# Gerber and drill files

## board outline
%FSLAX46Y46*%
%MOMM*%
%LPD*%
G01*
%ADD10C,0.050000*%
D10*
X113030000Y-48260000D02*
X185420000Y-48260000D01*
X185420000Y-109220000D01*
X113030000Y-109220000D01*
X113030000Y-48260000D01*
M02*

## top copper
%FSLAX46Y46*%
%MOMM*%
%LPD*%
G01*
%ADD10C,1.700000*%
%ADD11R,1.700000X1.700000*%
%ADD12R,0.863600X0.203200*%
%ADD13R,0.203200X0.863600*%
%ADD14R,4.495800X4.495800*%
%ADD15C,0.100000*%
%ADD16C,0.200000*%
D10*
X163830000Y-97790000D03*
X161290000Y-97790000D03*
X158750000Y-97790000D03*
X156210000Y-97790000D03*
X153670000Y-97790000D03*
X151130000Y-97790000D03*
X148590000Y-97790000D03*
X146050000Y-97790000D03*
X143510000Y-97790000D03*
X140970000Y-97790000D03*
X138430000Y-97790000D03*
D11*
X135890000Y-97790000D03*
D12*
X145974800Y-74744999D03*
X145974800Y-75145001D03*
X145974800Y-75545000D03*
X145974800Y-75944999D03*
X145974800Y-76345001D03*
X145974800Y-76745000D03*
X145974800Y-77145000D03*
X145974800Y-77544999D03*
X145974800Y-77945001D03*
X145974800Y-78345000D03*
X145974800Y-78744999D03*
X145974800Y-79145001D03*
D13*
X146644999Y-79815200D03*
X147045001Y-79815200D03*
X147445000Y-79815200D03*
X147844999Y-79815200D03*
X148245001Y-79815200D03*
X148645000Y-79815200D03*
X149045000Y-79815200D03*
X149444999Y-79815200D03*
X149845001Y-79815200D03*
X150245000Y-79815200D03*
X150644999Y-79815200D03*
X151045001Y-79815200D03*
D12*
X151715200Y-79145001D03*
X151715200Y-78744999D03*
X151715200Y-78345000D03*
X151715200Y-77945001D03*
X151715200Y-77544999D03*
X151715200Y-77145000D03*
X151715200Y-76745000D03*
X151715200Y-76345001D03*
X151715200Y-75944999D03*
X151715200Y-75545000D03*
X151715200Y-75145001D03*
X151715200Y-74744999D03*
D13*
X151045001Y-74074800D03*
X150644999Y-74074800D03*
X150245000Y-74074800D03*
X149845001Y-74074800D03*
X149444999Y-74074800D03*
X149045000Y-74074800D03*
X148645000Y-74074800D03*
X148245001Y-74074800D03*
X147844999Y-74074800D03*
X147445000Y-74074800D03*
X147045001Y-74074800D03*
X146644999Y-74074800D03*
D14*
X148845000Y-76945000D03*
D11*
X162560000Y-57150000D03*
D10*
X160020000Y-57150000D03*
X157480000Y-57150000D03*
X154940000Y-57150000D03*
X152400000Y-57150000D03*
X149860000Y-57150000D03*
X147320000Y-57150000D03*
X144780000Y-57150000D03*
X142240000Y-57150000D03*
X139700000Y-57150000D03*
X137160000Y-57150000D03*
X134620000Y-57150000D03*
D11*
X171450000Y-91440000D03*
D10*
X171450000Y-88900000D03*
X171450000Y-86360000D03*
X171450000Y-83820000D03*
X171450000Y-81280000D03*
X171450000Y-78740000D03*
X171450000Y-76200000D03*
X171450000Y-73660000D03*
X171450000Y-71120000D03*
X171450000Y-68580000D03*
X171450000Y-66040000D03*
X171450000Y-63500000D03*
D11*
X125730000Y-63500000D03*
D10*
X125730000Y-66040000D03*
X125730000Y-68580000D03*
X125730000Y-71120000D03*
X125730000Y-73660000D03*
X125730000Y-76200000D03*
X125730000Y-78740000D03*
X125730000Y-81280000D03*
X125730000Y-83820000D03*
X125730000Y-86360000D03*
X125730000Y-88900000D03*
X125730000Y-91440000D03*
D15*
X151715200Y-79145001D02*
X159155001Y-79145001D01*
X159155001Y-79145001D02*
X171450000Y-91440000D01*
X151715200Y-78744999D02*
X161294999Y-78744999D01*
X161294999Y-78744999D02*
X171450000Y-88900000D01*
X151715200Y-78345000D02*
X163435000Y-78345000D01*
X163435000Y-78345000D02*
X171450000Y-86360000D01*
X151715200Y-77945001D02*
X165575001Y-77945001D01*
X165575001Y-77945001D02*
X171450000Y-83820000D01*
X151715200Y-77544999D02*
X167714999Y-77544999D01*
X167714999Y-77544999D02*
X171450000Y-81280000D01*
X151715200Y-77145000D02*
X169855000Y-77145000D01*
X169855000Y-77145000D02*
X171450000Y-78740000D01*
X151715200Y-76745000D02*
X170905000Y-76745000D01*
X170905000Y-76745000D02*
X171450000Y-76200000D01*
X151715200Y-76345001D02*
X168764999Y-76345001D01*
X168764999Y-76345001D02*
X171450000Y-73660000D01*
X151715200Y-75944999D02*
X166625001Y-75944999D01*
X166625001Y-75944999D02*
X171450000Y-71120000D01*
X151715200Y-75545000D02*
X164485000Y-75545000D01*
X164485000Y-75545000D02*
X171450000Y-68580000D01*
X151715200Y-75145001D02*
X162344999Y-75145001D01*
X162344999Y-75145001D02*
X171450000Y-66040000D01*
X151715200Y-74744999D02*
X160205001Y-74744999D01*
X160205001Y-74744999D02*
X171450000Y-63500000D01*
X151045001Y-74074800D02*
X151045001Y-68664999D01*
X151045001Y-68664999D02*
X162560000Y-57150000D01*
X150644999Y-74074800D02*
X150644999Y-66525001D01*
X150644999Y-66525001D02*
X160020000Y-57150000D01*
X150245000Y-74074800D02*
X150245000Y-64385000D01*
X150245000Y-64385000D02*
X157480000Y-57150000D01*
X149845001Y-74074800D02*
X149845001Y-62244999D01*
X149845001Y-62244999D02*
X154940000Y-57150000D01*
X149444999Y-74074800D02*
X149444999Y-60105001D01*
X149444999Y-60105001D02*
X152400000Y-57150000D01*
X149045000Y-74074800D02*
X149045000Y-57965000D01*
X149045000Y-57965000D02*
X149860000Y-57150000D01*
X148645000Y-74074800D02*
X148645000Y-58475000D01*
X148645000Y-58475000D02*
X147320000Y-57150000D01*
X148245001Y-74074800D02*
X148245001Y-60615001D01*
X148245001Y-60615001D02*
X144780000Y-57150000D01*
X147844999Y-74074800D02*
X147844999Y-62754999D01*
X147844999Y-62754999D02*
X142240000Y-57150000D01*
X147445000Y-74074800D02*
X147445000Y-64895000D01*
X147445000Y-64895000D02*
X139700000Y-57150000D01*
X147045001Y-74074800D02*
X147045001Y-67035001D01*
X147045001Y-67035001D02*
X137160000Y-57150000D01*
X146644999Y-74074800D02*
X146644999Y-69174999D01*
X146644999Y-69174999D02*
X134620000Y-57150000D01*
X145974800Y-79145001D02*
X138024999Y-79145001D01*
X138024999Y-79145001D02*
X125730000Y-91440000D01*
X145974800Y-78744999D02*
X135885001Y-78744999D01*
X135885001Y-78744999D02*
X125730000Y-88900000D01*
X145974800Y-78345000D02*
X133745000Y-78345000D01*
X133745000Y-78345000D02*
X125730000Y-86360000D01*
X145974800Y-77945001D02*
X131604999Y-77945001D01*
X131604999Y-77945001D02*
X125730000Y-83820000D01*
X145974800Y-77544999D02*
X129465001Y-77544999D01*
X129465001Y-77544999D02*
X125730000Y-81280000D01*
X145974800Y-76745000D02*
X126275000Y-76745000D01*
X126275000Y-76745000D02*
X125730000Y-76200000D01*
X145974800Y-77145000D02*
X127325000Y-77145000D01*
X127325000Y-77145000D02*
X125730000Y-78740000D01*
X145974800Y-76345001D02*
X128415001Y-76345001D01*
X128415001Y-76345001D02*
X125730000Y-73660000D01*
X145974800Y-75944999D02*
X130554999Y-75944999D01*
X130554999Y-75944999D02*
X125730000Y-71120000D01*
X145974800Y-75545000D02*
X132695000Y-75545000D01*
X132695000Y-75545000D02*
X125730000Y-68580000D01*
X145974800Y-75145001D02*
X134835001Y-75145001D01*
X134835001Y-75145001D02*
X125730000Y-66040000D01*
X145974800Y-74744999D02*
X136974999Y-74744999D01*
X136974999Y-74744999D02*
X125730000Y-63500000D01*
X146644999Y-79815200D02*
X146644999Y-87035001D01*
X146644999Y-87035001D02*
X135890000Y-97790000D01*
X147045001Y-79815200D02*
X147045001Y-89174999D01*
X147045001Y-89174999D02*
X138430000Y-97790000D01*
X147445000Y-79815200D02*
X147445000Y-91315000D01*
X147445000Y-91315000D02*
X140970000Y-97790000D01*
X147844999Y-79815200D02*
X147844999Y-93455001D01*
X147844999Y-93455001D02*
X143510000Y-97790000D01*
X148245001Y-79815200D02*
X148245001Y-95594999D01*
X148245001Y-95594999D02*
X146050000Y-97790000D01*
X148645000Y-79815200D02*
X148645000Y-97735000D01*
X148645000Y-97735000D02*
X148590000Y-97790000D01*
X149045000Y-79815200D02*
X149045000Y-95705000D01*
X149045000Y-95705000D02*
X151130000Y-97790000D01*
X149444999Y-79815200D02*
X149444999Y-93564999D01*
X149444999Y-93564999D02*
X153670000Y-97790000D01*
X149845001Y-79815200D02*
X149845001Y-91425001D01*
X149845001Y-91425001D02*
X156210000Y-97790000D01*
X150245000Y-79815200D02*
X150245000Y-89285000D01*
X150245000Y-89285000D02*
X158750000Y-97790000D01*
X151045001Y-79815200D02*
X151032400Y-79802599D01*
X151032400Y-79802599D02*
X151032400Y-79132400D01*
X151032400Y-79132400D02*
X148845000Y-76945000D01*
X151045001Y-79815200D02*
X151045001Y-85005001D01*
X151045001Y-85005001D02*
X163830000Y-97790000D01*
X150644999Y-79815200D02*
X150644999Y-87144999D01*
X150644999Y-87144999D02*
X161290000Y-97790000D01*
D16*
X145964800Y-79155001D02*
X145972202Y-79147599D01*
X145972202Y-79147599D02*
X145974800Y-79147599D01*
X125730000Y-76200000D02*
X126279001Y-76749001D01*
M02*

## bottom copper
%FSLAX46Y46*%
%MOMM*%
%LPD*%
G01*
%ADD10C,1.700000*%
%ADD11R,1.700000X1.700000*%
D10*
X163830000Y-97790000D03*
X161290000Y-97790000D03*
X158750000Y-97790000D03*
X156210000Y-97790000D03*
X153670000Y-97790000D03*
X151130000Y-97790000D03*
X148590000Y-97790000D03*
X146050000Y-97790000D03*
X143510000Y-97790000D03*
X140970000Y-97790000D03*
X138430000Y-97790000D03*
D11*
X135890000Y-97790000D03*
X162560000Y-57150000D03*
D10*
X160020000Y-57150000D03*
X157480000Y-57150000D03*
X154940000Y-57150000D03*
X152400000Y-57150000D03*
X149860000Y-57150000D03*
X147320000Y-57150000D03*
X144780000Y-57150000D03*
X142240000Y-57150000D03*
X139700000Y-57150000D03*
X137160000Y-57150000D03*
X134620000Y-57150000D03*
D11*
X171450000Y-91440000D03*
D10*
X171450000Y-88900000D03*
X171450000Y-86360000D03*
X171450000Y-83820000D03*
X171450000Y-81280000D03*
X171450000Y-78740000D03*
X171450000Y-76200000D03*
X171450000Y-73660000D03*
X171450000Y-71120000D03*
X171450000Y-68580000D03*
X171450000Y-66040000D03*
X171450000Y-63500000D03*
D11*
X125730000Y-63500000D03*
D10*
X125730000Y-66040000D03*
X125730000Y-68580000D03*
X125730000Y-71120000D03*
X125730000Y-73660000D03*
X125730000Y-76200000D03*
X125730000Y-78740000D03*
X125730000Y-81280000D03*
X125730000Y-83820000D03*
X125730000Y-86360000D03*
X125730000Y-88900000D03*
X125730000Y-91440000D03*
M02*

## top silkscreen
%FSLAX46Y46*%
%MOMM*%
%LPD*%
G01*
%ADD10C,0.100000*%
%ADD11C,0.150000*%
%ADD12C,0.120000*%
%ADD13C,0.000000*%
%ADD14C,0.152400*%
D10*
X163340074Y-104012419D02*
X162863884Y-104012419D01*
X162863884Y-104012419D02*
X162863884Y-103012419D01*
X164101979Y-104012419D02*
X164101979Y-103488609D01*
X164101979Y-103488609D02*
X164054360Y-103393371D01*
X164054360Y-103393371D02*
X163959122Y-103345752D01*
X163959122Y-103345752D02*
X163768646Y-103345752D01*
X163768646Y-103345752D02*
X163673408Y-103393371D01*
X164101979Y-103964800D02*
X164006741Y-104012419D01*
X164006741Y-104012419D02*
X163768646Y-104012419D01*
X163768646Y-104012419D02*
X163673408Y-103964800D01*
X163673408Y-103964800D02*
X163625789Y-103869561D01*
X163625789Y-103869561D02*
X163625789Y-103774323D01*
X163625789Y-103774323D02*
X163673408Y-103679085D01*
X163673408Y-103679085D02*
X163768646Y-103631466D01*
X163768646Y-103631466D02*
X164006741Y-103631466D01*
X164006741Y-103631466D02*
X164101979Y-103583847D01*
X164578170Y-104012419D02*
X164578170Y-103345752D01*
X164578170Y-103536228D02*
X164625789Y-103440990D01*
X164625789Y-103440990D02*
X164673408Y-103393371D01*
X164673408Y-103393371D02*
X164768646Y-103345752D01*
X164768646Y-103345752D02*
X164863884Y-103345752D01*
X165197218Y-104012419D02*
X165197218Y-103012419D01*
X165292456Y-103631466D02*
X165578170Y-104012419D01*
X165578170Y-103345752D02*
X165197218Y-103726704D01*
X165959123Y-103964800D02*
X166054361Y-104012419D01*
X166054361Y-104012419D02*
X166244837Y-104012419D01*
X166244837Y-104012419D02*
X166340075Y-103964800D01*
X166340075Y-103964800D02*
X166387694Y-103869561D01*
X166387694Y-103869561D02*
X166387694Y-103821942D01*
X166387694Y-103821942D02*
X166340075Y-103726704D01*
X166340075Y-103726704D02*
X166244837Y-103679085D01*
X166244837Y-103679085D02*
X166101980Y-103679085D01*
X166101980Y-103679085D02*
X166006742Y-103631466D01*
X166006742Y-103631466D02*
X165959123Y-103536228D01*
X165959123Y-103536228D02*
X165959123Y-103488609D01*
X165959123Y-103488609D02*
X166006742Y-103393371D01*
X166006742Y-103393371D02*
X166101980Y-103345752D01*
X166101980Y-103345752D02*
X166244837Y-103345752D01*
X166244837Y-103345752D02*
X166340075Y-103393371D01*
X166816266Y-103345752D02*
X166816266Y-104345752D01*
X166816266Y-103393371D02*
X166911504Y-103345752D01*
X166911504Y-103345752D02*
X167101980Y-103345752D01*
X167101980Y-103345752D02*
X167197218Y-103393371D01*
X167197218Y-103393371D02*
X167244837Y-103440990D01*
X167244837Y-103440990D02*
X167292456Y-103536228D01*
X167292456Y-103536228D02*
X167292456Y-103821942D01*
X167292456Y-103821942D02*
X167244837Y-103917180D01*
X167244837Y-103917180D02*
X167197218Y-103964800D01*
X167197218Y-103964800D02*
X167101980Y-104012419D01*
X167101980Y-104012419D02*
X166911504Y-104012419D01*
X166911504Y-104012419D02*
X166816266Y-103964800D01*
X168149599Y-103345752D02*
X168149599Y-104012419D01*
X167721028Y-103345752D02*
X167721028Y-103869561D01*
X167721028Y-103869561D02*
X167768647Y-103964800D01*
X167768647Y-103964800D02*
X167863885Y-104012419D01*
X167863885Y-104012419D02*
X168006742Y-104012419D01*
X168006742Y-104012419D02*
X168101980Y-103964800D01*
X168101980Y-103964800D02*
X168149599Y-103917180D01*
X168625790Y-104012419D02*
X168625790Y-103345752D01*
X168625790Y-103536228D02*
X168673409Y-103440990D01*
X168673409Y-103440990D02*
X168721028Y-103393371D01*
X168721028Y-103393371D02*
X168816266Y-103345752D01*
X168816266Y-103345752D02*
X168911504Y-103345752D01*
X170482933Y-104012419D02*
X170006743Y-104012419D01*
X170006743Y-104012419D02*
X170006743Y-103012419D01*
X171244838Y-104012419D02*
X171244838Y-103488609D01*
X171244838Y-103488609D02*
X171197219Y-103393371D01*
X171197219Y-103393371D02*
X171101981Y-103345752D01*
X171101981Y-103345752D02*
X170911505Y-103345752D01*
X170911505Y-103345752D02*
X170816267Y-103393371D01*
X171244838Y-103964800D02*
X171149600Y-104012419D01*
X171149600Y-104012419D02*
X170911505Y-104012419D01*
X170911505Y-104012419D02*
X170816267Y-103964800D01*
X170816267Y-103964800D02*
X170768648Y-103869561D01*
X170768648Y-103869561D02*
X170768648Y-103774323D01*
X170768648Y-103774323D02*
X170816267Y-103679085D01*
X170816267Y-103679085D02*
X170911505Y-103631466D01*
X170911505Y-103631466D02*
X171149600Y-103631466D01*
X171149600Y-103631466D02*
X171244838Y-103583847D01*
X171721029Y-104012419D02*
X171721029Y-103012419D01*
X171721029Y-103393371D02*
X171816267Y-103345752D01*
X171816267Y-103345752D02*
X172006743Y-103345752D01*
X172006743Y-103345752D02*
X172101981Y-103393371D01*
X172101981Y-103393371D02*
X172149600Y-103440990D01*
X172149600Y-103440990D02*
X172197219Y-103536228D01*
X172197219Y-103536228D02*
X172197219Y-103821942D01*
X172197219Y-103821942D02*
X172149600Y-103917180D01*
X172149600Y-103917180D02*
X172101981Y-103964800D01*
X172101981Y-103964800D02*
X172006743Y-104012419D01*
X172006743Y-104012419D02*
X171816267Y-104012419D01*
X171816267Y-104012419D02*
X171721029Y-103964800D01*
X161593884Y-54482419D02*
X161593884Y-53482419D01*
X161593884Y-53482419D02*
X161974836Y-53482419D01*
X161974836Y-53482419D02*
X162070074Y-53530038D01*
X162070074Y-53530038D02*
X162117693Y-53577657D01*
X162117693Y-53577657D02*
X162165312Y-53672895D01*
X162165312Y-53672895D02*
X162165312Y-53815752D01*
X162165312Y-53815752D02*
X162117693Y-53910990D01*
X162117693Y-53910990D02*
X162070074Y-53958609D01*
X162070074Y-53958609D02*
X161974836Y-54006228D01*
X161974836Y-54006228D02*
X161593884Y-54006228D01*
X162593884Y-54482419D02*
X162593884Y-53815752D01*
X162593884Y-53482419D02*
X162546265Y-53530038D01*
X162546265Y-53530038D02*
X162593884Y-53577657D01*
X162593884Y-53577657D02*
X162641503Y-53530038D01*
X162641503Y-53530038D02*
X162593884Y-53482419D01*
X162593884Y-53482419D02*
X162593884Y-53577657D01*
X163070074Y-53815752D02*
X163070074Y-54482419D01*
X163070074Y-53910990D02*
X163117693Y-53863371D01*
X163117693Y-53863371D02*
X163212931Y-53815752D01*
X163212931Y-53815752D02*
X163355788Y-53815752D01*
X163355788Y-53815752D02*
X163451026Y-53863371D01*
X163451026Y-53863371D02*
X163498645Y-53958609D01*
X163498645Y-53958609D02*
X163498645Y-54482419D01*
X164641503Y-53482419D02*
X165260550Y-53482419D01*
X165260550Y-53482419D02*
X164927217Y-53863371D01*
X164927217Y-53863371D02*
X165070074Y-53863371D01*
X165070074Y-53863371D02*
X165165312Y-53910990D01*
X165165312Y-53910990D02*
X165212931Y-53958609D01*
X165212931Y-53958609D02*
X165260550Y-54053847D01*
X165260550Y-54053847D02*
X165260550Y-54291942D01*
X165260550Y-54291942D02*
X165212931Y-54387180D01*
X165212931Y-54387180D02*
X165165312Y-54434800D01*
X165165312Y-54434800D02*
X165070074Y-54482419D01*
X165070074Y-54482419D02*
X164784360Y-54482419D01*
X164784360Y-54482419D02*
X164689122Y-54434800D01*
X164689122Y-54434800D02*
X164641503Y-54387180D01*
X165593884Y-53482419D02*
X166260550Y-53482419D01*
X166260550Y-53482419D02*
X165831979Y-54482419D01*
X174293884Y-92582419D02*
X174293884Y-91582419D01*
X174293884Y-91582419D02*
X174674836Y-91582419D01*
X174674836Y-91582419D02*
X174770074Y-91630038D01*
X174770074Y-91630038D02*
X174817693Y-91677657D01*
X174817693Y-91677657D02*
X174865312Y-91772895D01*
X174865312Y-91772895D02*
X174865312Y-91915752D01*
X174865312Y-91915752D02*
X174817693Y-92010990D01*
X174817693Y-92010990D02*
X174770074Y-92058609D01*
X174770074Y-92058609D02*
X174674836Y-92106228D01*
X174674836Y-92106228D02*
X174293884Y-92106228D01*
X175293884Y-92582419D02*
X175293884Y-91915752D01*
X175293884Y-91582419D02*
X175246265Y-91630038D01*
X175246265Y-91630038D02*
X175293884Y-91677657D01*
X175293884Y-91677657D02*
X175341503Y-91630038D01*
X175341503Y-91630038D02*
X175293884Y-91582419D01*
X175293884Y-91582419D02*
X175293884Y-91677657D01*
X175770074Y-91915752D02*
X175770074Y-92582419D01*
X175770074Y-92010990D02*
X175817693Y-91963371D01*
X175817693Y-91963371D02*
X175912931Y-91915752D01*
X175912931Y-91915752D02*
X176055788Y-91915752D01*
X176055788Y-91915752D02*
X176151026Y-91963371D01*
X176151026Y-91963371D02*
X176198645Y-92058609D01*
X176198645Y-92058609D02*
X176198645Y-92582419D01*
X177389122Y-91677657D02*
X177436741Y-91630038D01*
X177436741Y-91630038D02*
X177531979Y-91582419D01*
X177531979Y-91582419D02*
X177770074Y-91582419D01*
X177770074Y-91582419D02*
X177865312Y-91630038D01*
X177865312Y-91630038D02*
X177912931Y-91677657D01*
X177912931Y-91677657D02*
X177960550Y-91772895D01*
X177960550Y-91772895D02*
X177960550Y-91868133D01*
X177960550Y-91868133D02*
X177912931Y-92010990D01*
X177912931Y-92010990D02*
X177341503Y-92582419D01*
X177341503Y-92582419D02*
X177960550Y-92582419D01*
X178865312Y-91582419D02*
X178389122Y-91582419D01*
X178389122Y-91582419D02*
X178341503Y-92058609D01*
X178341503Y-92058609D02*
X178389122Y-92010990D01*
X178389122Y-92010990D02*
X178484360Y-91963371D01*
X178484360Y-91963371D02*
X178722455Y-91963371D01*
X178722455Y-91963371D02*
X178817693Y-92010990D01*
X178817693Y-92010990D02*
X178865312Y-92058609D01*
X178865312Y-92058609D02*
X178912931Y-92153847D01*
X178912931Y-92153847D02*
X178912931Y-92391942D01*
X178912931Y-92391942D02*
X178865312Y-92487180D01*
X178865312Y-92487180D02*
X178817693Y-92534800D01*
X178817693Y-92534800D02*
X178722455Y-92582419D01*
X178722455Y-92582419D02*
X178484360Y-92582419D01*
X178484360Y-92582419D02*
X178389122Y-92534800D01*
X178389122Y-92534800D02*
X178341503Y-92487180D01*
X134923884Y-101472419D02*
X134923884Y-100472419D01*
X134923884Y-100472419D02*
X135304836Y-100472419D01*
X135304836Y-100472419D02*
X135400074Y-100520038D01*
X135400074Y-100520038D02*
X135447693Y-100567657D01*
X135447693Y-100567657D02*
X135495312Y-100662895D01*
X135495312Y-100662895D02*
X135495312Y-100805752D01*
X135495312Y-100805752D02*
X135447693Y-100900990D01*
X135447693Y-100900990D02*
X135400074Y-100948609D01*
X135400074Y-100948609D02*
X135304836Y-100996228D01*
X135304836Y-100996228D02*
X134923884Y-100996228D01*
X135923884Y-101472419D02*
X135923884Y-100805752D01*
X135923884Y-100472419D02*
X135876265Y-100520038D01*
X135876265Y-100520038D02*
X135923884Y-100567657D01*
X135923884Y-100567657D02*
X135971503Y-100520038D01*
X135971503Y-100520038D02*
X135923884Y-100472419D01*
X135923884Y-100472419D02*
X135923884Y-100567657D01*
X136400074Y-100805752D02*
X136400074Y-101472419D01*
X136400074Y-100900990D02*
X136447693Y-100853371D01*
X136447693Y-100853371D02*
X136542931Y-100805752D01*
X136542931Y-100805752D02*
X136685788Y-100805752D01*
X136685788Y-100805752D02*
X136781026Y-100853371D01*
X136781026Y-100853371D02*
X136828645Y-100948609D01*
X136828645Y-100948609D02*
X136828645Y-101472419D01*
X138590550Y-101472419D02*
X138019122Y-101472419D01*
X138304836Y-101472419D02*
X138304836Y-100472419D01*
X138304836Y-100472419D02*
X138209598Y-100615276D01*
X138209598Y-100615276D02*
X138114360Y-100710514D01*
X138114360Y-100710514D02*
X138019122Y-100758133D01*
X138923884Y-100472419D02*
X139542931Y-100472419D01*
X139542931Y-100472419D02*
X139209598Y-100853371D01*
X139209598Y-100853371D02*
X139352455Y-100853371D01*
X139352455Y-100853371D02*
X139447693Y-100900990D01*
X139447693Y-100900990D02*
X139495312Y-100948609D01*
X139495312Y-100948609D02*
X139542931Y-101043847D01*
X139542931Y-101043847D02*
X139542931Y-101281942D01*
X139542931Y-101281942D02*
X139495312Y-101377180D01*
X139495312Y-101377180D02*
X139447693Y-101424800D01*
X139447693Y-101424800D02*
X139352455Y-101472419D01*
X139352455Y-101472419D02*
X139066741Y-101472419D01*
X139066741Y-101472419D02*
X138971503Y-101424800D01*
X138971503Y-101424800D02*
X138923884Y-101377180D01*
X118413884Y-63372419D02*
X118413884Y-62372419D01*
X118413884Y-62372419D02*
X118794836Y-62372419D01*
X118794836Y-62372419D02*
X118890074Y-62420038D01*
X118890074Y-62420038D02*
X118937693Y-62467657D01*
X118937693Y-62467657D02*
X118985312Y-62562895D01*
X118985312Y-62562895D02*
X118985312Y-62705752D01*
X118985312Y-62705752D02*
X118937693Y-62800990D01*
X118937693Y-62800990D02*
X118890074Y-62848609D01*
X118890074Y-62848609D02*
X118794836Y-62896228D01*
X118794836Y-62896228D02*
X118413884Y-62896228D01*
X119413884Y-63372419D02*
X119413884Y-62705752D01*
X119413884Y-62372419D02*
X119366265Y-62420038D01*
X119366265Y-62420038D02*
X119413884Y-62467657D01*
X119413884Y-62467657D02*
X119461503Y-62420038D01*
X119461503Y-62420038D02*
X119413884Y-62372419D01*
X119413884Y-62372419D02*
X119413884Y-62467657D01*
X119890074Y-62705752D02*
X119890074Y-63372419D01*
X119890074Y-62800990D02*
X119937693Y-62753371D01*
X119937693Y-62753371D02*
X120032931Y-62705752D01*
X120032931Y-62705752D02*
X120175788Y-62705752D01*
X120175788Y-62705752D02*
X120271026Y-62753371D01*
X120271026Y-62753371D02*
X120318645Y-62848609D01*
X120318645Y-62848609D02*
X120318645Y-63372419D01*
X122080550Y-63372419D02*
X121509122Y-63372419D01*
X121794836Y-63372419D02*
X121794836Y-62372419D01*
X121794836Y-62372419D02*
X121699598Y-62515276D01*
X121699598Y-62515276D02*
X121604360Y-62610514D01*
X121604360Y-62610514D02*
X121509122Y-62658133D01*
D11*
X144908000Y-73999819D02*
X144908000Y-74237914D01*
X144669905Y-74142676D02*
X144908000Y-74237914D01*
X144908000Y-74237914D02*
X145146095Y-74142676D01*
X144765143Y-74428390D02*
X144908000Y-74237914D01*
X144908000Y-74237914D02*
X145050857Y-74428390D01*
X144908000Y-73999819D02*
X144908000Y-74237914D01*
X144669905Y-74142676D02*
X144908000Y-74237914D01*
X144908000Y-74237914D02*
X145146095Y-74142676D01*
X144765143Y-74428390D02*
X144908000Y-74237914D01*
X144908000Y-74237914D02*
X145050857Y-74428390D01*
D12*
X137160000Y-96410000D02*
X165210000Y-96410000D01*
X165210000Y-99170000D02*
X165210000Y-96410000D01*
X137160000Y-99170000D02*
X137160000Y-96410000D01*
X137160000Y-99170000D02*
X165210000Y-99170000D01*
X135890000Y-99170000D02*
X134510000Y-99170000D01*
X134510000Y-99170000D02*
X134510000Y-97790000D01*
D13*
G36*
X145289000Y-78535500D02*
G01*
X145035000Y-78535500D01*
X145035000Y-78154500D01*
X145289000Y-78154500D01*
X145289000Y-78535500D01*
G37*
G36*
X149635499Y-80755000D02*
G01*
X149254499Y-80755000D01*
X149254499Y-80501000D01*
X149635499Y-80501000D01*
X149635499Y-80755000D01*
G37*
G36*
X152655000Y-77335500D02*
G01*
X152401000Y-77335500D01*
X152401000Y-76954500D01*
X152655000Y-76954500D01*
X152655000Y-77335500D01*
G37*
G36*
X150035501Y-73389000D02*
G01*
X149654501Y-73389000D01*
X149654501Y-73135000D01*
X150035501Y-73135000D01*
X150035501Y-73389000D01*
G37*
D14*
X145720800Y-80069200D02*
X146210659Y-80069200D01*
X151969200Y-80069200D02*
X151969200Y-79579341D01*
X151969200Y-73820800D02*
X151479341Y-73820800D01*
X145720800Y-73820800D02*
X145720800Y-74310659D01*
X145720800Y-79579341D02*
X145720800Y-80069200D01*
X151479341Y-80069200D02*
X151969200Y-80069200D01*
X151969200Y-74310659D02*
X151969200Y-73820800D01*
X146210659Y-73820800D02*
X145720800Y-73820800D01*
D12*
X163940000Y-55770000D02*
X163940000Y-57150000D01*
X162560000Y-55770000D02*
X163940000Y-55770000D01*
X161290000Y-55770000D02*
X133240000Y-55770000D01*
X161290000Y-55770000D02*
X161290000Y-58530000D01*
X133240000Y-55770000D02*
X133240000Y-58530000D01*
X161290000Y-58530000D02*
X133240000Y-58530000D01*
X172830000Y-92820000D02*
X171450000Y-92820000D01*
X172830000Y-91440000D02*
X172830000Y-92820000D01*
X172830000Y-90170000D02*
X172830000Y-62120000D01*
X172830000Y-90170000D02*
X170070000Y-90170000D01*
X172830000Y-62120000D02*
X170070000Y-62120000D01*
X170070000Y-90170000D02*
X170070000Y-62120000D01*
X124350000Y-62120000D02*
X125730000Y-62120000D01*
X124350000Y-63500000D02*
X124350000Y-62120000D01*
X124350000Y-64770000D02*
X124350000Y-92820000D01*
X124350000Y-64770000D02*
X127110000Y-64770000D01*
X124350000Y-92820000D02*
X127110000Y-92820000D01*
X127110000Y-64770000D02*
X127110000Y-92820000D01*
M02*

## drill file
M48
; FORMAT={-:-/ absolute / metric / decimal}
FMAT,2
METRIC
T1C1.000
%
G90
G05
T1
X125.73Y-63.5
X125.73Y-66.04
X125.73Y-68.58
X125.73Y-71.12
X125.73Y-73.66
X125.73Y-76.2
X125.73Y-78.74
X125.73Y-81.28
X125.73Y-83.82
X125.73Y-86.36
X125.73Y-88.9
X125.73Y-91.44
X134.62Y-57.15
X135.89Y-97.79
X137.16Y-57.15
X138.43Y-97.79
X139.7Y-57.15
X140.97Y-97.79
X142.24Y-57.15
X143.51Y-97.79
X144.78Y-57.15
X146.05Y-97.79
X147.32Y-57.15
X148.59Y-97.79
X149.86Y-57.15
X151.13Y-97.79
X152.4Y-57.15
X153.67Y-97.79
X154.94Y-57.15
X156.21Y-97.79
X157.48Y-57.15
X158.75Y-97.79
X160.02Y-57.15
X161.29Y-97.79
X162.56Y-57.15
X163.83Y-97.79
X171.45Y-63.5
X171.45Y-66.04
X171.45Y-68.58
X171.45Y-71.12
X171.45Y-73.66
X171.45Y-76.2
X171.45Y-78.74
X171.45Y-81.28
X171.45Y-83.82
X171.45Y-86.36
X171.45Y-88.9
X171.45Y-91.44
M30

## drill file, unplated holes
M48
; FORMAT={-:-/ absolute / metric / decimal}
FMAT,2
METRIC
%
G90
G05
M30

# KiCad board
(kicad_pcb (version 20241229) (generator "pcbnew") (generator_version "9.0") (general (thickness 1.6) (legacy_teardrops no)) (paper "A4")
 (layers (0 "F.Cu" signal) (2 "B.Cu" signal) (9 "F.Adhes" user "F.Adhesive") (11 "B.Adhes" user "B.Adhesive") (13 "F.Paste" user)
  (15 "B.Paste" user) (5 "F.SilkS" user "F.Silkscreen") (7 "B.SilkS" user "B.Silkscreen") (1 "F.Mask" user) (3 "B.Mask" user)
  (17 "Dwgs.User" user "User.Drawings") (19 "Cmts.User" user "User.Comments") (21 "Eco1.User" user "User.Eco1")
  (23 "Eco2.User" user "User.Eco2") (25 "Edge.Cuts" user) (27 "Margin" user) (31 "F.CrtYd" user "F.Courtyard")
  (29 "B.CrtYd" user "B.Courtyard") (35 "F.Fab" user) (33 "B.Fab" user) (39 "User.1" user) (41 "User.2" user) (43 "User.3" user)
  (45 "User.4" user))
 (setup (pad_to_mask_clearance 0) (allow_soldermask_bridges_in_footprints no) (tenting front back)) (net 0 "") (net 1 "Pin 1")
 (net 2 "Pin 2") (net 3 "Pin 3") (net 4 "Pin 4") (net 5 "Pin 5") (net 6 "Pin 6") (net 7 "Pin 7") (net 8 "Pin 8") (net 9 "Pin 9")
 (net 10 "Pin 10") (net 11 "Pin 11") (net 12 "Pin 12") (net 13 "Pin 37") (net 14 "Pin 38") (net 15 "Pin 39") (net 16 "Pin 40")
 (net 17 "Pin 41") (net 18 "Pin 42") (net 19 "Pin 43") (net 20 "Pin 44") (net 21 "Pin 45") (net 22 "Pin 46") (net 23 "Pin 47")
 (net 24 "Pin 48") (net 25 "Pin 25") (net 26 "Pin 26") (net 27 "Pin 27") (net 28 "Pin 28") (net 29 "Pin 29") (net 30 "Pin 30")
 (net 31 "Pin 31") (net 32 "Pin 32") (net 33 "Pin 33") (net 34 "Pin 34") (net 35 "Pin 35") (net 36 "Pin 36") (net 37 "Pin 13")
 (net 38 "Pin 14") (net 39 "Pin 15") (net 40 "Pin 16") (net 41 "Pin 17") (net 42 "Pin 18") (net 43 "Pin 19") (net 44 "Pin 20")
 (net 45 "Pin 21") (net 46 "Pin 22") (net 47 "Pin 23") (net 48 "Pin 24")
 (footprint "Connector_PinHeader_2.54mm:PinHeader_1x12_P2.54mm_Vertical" (layer "F.Cu") (at 125.73 63.5)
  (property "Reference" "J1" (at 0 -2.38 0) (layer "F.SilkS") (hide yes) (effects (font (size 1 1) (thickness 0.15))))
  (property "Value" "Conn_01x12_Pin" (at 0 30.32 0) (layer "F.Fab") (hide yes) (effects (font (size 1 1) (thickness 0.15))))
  (fp_line (start -1.38 -1.38) (end 0 -1.38) (stroke (width 0.12) (type solid)) (layer "F.SilkS"))
  (fp_line (start -1.38 0) (end -1.38 -1.38) (stroke (width 0.12) (type solid)) (layer "F.SilkS"))
  (fp_line (start -1.38 1.27) (end -1.38 29.32) (stroke (width 0.12) (type solid)) (layer "F.SilkS"))
  (fp_line (start -1.38 1.27) (end 1.38 1.27) (stroke (width 0.12) (type solid)) (layer "F.SilkS"))
  (fp_line (start -1.38 29.32) (end 1.38 29.32) (stroke (width 0.12) (type solid)) (layer "F.SilkS"))
  (fp_line (start 1.38 1.27) (end 1.38 29.32) (stroke (width 0.12) (type solid)) (layer "F.SilkS"))
  (pad "1" thru_hole rect (at 0 0) (size 1.7 1.7) (drill 1) (layers "*.Cu" "*.Mask") (remove_unused_layers no) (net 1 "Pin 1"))
  (pad "2" thru_hole circle (at 0 2.54) (size 1.7 1.7) (drill 1) (layers "*.Cu" "*.Mask") (remove_unused_layers no) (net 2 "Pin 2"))
  (pad "3" thru_hole circle (at 0 5.08) (size 1.7 1.7) (drill 1) (layers "*.Cu" "*.Mask") (remove_unused_layers no) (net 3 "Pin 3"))
  (pad "4" thru_hole circle (at 0 7.62) (size 1.7 1.7) (drill 1) (layers "*.Cu" "*.Mask") (remove_unused_layers no) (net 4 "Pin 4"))
  (pad "5" thru_hole circle (at 0 10.16) (size 1.7 1.7) (drill 1) (layers "*.Cu" "*.Mask") (remove_unused_layers no) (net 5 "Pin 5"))
  (pad "6" thru_hole circle (at 0 12.7) (size 1.7 1.7) (drill 1) (layers "*.Cu" "*.Mask") (remove_unused_layers no) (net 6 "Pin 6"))
  (pad "7" thru_hole circle (at 0 15.24) (size 1.7 1.7) (drill 1) (layers "*.Cu" "*.Mask") (remove_unused_layers no) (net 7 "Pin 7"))
  (pad "8" thru_hole circle (at 0 17.78) (size 1.7 1.7) (drill 1) (layers "*.Cu" "*.Mask") (remove_unused_layers no) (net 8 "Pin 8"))
  (pad "9" thru_hole circle (at 0 20.32) (size 1.7 1.7) (drill 1) (layers "*.Cu" "*.Mask") (remove_unused_layers no) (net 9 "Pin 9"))
  (pad "10" thru_hole circle (at 0 22.86) (size 1.7 1.7) (drill 1) (layers "*.Cu" "*.Mask") (remove_unused_layers no) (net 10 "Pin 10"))
  (pad "11" thru_hole circle (at 0 25.4) (size 1.7 1.7) (drill 1) (layers "*.Cu" "*.Mask") (remove_unused_layers no) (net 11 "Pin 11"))
  (pad "12" thru_hole circle (at 0 27.94) (size 1.7 1.7) (drill 1) (layers "*.Cu" "*.Mask") (remove_unused_layers no) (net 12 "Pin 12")))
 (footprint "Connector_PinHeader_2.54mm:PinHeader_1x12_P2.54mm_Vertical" (layer "F.Cu") (at 162.56 57.15 -90)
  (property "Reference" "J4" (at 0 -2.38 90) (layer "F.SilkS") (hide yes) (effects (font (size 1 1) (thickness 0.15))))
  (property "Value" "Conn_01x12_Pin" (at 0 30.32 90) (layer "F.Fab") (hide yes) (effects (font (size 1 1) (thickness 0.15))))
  (fp_line (start -1.38 29.32) (end 1.38 29.32) (stroke (width 0.12) (type solid)) (layer "F.SilkS"))
  (fp_line (start -1.38 1.27) (end -1.38 29.32) (stroke (width 0.12) (type solid)) (layer "F.SilkS"))
  (fp_line (start -1.38 1.27) (end 1.38 1.27) (stroke (width 0.12) (type solid)) (layer "F.SilkS"))
  (fp_line (start 1.38 1.27) (end 1.38 29.32) (stroke (width 0.12) (type solid)) (layer "F.SilkS"))
  (fp_line (start -1.38 0) (end -1.38 -1.38) (stroke (width 0.12) (type solid)) (layer "F.SilkS"))
  (fp_line (start -1.38 -1.38) (end 0 -1.38) (stroke (width 0.12) (type solid)) (layer "F.SilkS"))
  (pad "1" thru_hole rect (at 0 0 270) (size 1.7 1.7) (drill 1) (layers "*.Cu" "*.Mask") (remove_unused_layers no) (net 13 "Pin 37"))
  (pad "2" thru_hole circle (at 0 2.54 270) (size 1.7 1.7) (drill 1) (layers "*.Cu" "*.Mask") (remove_unused_layers no) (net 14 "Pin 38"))
  (pad "3" thru_hole circle (at 0 5.08 270) (size 1.7 1.7) (drill 1) (layers "*.Cu" "*.Mask") (remove_unused_layers no) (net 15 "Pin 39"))
  (pad "4" thru_hole circle (at 0 7.62 270) (size 1.7 1.7) (drill 1) (layers "*.Cu" "*.Mask") (remove_unused_layers no) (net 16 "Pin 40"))
  (pad "5" thru_hole circle (at 0 10.16 270) (size 1.7 1.7) (drill 1) (layers "*.Cu" "*.Mask") (remove_unused_layers no) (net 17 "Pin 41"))
  (pad "6" thru_hole circle (at 0 12.7 270) (size 1.7 1.7) (drill 1) (layers "*.Cu" "*.Mask") (remove_unused_layers no) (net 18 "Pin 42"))
  (pad "7" thru_hole circle (at 0 15.24 270) (size 1.7 1.7) (drill 1) (layers "*.Cu" "*.Mask") (remove_unused_layers no) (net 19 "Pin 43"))
  (pad "8" thru_hole circle (at 0 17.78 270) (size 1.7 1.7) (drill 1) (layers "*.Cu" "*.Mask") (remove_unused_layers no) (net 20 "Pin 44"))
  (pad "9" thru_hole circle (at 0 20.32 270) (size 1.7 1.7) (drill 1) (layers "*.Cu" "*.Mask") (remove_unused_layers no) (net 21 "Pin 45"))
  (pad "10" thru_hole circle (at 0 22.86 270) (size 1.7 1.7) (drill 1) (layers "*.Cu" "*.Mask") (remove_unused_layers no) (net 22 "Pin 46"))
  (pad "11" thru_hole circle (at 0 25.4 270) (size 1.7 1.7) (drill 1) (layers "*.Cu" "*.Mask") (remove_unused_layers no) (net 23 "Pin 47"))
  (pad "12" thru_hole circle (at 0 27.94 270) (size 1.7 1.7) (drill 1) (layers "*.Cu" "*.Mask") (remove_unused_layers no) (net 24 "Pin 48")))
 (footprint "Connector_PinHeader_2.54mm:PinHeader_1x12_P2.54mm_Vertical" (layer "F.Cu") (at 171.45 91.44 180)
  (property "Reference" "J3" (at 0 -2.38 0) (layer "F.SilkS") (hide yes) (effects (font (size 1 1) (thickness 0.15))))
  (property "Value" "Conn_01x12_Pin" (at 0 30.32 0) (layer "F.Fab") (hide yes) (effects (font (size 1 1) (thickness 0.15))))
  (fp_line (start 1.38 1.27) (end 1.38 29.32) (stroke (width 0.12) (type solid)) (layer "F.SilkS"))
  (fp_line (start -1.38 29.32) (end 1.38 29.32) (stroke (width 0.12) (type solid)) (layer "F.SilkS"))
  (fp_line (start -1.38 1.27) (end 1.38 1.27) (stroke (width 0.12) (type solid)) (layer "F.SilkS"))
  (fp_line (start -1.38 1.27) (end -1.38 29.32) (stroke (width 0.12) (type solid)) (layer "F.SilkS"))
  (fp_line (start -1.38 0) (end -1.38 -1.38) (stroke (width 0.12) (type solid)) (layer "F.SilkS"))
  (fp_line (start -1.38 -1.38) (end 0 -1.38) (stroke (width 0.12) (type solid)) (layer "F.SilkS"))
  (pad "1" thru_hole rect (at 0 0 180) (size 1.7 1.7) (drill 1) (layers "*.Cu" "*.Mask") (remove_unused_layers no) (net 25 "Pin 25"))
  (pad "2" thru_hole circle (at 0 2.54 180) (size 1.7 1.7) (drill 1) (layers "*.Cu" "*.Mask") (remove_unused_layers no) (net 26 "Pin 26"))
  (pad "3" thru_hole circle (at 0 5.08 180) (size 1.7 1.7) (drill 1) (layers "*.Cu" "*.Mask") (remove_unused_layers no) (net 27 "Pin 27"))
  (pad "4" thru_hole circle (at 0 7.62 180) (size 1.7 1.7) (drill 1) (layers "*.Cu" "*.Mask") (remove_unused_layers no) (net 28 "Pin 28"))
  (pad "5" thru_hole circle (at 0 10.16 180) (size 1.7 1.7) (drill 1) (layers "*.Cu" "*.Mask") (remove_unused_layers no) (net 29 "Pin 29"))
  (pad "6" thru_hole circle (at 0 12.7 180) (size 1.7 1.7) (drill 1) (layers "*.Cu" "*.Mask") (remove_unused_layers no) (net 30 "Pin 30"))
  (pad "7" thru_hole circle (at 0 15.24 180) (size 1.7 1.7) (drill 1) (layers "*.Cu" "*.Mask") (remove_unused_layers no) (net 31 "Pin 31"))
  (pad "8" thru_hole circle (at 0 17.78 180) (size 1.7 1.7) (drill 1) (layers "*.Cu" "*.Mask") (remove_unused_layers no) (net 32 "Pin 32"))
  (pad "9" thru_hole circle (at 0 20.32 180) (size 1.7 1.7) (drill 1) (layers "*.Cu" "*.Mask") (remove_unused_layers no) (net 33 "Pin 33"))
  (pad "10" thru_hole circle (at 0 22.86 180) (size 1.7 1.7) (drill 1) (layers "*.Cu" "*.Mask") (remove_unused_layers no) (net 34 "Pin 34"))
  (pad "11" thru_hole circle (at 0 25.4 180) (size 1.7 1.7) (drill 1) (layers "*.Cu" "*.Mask") (remove_unused_layers no) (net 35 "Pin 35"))
  (pad "12" thru_hole circle (at 0 27.94 180) (size 1.7 1.7) (drill 1) (layers "*.Cu" "*.Mask") (remove_unused_layers no) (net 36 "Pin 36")))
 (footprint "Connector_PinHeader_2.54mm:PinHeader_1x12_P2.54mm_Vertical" (layer "F.Cu") (at 135.89 97.79 90)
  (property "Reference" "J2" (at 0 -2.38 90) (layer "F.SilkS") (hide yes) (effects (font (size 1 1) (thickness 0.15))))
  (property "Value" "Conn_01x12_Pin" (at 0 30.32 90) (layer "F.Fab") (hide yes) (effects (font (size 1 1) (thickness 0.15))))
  (fp_line (start -1.38 -1.38) (end 0 -1.38) (stroke (width 0.12) (type solid)) (layer "F.SilkS"))
  (fp_line (start -1.38 0) (end -1.38 -1.38) (stroke (width 0.12) (type solid)) (layer "F.SilkS"))
  (fp_line (start 1.38 1.27) (end 1.38 29.32) (stroke (width 0.12) (type solid)) (layer "F.SilkS"))
  (fp_line (start -1.38 1.27) (end 1.38 1.27) (stroke (width 0.12) (type solid)) (layer "F.SilkS"))
  (fp_line (start -1.38 1.27) (end -1.38 29.32) (stroke (width 0.12) (type solid)) (layer "F.SilkS"))
  (fp_line (start -1.38 29.32) (end 1.38 29.32) (stroke (width 0.12) (type solid)) (layer "F.SilkS"))
  (pad "1" thru_hole rect (at 0 0 90) (size 1.7 1.7) (drill 1) (layers "*.Cu" "*.Mask") (remove_unused_layers no) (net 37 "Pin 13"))
  (pad "2" thru_hole circle (at 0 2.54 90) (size 1.7 1.7) (drill 1) (layers "*.Cu" "*.Mask") (remove_unused_layers no) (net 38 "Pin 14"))
  (pad "3" thru_hole circle (at 0 5.08 90) (size 1.7 1.7) (drill 1) (layers "*.Cu" "*.Mask") (remove_unused_layers no) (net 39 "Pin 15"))
  (pad "4" thru_hole circle (at 0 7.62 90) (size 1.7 1.7) (drill 1) (layers "*.Cu" "*.Mask") (remove_unused_layers no) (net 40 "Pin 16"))
  (pad "5" thru_hole circle (at 0 10.16 90) (size 1.7 1.7) (drill 1) (layers "*.Cu" "*.Mask") (remove_unused_layers no) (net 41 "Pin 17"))
  (pad "6" thru_hole circle (at 0 12.7 90) (size 1.7 1.7) (drill 1) (layers "*.Cu" "*.Mask") (remove_unused_layers no) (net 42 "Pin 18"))
  (pad "7" thru_hole circle (at 0 15.24 90) (size 1.7 1.7) (drill 1) (layers "*.Cu" "*.Mask") (remove_unused_layers no) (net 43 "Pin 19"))
  (pad "8" thru_hole circle (at 0 17.78 90) (size 1.7 1.7) (drill 1) (layers "*.Cu" "*.Mask") (remove_unused_layers no) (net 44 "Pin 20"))
  (pad "9" thru_hole circle (at 0 20.32 90) (size 1.7 1.7) (drill 1) (layers "*.Cu" "*.Mask") (remove_unused_layers no) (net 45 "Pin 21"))
  (pad "10" thru_hole circle (at 0 22.86 90) (size 1.7 1.7) (drill 1) (layers "*.Cu" "*.Mask") (remove_unused_layers no) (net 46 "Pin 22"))
  (pad "11" thru_hole circle (at 0 25.4 90) (size 1.7 1.7) (drill 1) (layers "*.Cu" "*.Mask") (remove_unused_layers no) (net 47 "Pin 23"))
  (pad "12" thru_hole circle (at 0 27.94 90) (size 1.7 1.7) (drill 1) (layers "*.Cu" "*.Mask") (remove_unused_layers no) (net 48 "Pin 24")))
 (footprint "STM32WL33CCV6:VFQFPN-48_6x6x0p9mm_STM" (layer "F.Cu") (at 148.845 76.945)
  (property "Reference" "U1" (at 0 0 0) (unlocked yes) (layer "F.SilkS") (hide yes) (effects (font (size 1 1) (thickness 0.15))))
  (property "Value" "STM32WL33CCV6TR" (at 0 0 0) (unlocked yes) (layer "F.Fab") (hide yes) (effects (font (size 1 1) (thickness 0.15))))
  (fp_line (start -3.1242 -3.1242) (end -3.1242 -2.634341) (stroke (width 0.1524) (type solid)) (layer "F.SilkS"))
  (fp_line (start -3.1242 2.634341) (end -3.1242 3.1242) (stroke (width 0.1524) (type solid)) (layer "F.SilkS"))
  (fp_line (start -3.1242 3.1242) (end -2.634341 3.1242) (stroke (width 0.1524) (type solid)) (layer "F.SilkS"))
  (fp_line (start -2.634341 -3.1242) (end -3.1242 -3.1242) (stroke (width 0.1524) (type solid)) (layer "F.SilkS"))
  (fp_line (start 2.634341 3.1242) (end 3.1242 3.1242) (stroke (width 0.1524) (type solid)) (layer "F.SilkS"))
  (fp_line (start 3.1242 -3.1242) (end 2.634341 -3.1242) (stroke (width 0.1524) (type solid)) (layer "F.SilkS"))
  (fp_line (start 3.1242 -2.634341) (end 3.1242 -3.1242) (stroke (width 0.1524) (type solid)) (layer "F.SilkS"))
  (fp_line (start 3.1242 3.1242) (end 3.1242 2.634341) (stroke (width 0.1524) (type solid)) (layer "F.SilkS"))
  (fp_poly
   (pts (xy -3.81 1.2095) (xy -3.81 1.5905) (xy -3.556 1.5905) (xy -3.556 1.2095)) (stroke (width 0) (type solid)) (fill yes)
   (layer "F.SilkS"))
  (fp_poly
   (pts (xy 0.409499 3.556) (xy 0.409499 3.81) (xy 0.790499 3.81) (xy 0.790499 3.556)) (stroke (width 0) (type solid)) (fill yes)
   (layer "F.SilkS"))
  (fp_poly
   (pts (xy 0.809501 -3.556) (xy 0.809501 -3.81) (xy 1.190501 -3.81) (xy 1.190501 -3.556)) (stroke (width 0) (type solid)) (fill yes)
   (layer "F.SilkS"))
  (fp_poly
   (pts (xy 3.81 0.0095) (xy 3.81 0.3905) (xy 3.556 0.3905) (xy 3.556 0.0095)) (stroke (width 0) (type solid)) (fill yes) (layer "F.SilkS"))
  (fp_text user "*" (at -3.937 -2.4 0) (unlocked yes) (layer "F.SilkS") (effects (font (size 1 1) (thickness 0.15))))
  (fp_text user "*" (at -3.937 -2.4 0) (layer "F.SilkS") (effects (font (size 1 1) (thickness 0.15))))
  (pad "1" smd rect (at -2.8702 -2.200001 90) (size 0.2032 0.8636) (layers "F.Cu" "F.Mask" "F.Paste") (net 1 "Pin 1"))
  (pad "2" smd rect (at -2.8702 -1.799999 90) (size 0.2032 0.8636) (layers "F.Cu" "F.Mask" "F.Paste") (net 2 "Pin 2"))
  (pad "3" smd rect (at -2.8702 -1.4 90) (size 0.2032 0.8636) (layers "F.Cu" "F.Mask" "F.Paste") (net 3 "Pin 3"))
  (pad "4" smd rect (at -2.8702 -1.000001 90) (size 0.2032 0.8636) (layers "F.Cu" "F.Mask" "F.Paste") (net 4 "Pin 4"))
  (pad "5" smd rect (at -2.8702 -0.599999 90) (size 0.2032 0.8636) (layers "F.Cu" "F.Mask" "F.Paste") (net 5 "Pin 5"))
  (pad "6" smd rect (at -2.8702 -0.2 90) (size 0.2032 0.8636) (layers "F.Cu" "F.Mask" "F.Paste") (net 6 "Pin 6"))
  (pad "7" smd rect (at -2.8702 0.2 90) (size 0.2032 0.8636) (layers "F.Cu" "F.Mask" "F.Paste") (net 7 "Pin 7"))
  (pad "8" smd rect (at -2.8702 0.599999 90) (size 0.2032 0.8636) (layers "F.Cu" "F.Mask" "F.Paste") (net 8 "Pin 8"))
  (pad "9" smd rect (at -2.8702 1.000001 90) (size 0.2032 0.8636) (layers "F.Cu" "F.Mask" "F.Paste") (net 9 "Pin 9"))
  (pad "10" smd rect (at -2.8702 1.4 90) (size 0.2032 0.8636) (layers "F.Cu" "F.Mask" "F.Paste") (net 10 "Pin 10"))
  (pad "11" smd rect (at -2.8702 1.799999 90) (size 0.2032 0.8636) (layers "F.Cu" "F.Mask" "F.Paste") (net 11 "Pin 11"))
  (pad "12" smd rect (at -2.8702 2.200001 90) (size 0.2032 0.8636) (layers "F.Cu" "F.Mask" "F.Paste") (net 12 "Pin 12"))
  (pad "13" smd rect (at -2.200001 2.8702) (size 0.2032 0.8636) (layers "F.Cu" "F.Mask" "F.Paste") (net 37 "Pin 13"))
  (pad "14" smd rect (at -1.799999 2.8702) (size 0.2032 0.8636) (layers "F.Cu" "F.Mask" "F.Paste") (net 38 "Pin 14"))
  (pad "15" smd rect (at -1.4 2.8702) (size 0.2032 0.8636) (layers "F.Cu" "F.Mask" "F.Paste") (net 39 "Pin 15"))
  (pad "16" smd rect (at -1.000001 2.8702) (size 0.2032 0.8636) (layers "F.Cu" "F.Mask" "F.Paste") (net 40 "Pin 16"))
  (pad "17" smd rect (at -0.599999 2.8702) (size 0.2032 0.8636) (layers "F.Cu" "F.Mask" "F.Paste") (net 41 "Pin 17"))
  (pad "18" smd rect (at -0.2 2.8702) (size 0.2032 0.8636) (layers "F.Cu" "F.Mask" "F.Paste") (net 42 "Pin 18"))
  (pad "19" smd rect (at 0.2 2.8702) (size 0.2032 0.8636) (layers "F.Cu" "F.Mask" "F.Paste") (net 43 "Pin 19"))
  (pad "20" smd rect (at 0.599999 2.8702) (size 0.2032 0.8636) (layers "F.Cu" "F.Mask" "F.Paste") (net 44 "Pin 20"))
  (pad "21" smd rect (at 1.000001 2.8702) (size 0.2032 0.8636) (layers "F.Cu" "F.Mask" "F.Paste") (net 45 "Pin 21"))
  (pad "22" smd rect (at 1.4 2.8702) (size 0.2032 0.8636) (layers "F.Cu" "F.Mask" "F.Paste") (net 46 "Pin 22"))
  (pad "23" smd rect (at 1.799999 2.8702) (size 0.2032 0.8636) (layers "F.Cu" "F.Mask" "F.Paste") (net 47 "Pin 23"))
  (pad "24" smd rect (at 2.200001 2.8702) (size 0.2032 0.8636) (layers "F.Cu" "F.Mask" "F.Paste") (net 48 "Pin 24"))
  (pad "25" smd rect (at 2.8702 2.200001 90) (size 0.2032 0.8636) (layers "F.Cu" "F.Mask" "F.Paste") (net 25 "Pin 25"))
  (pad "26" smd rect (at 2.8702 1.799999 90) (size 0.2032 0.8636) (layers "F.Cu" "F.Mask" "F.Paste") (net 26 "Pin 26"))
  (pad "27" smd rect (at 2.8702 1.4 90) (size 0.2032 0.8636) (layers "F.Cu" "F.Mask" "F.Paste") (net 27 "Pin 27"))
  (pad "28" smd rect (at 2.8702 1.000001 90) (size 0.2032 0.8636) (layers "F.Cu" "F.Mask" "F.Paste") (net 28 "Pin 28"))
  (pad "29" smd rect (at 2.8702 0.599999 90) (size 0.2032 0.8636) (layers "F.Cu" "F.Mask" "F.Paste") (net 29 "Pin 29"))
  (pad "30" smd rect (at 2.8702 0.2 90) (size 0.2032 0.8636) (layers "F.Cu" "F.Mask" "F.Paste") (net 30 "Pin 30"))
  (pad "31" smd rect (at 2.8702 -0.2 90) (size 0.2032 0.8636) (layers "F.Cu" "F.Mask" "F.Paste") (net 31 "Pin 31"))
  (pad "32" smd rect (at 2.8702 -0.599999 90) (size 0.2032 0.8636) (layers "F.Cu" "F.Mask" "F.Paste") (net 32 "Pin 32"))
  (pad "33" smd rect (at 2.8702 -1.000001 90) (size 0.2032 0.8636) (layers "F.Cu" "F.Mask" "F.Paste") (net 33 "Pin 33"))
  (pad "34" smd rect (at 2.8702 -1.4 90) (size 0.2032 0.8636) (layers "F.Cu" "F.Mask" "F.Paste") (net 34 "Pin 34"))
  (pad "35" smd rect (at 2.8702 -1.799999 90) (size 0.2032 0.8636) (layers "F.Cu" "F.Mask" "F.Paste") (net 35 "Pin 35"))
  (pad "36" smd rect (at 2.8702 -2.200001 90) (size 0.2032 0.8636) (layers "F.Cu" "F.Mask" "F.Paste") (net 36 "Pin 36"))
  (pad "37" smd rect (at 2.200001 -2.8702) (size 0.2032 0.8636) (layers "F.Cu" "F.Mask" "F.Paste") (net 13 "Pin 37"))
  (pad "38" smd rect (at 1.799999 -2.8702) (size 0.2032 0.8636) (layers "F.Cu" "F.Mask" "F.Paste") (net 14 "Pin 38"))
  (pad "39" smd rect (at 1.4 -2.8702) (size 0.2032 0.8636) (layers "F.Cu" "F.Mask" "F.Paste") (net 15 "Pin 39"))
  (pad "40" smd rect (at 1.000001 -2.8702) (size 0.2032 0.8636) (layers "F.Cu" "F.Mask" "F.Paste") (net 16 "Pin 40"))
  (pad "41" smd rect (at 0.599999 -2.8702) (size 0.2032 0.8636) (layers "F.Cu" "F.Mask" "F.Paste") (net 17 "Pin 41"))
  (pad "42" smd rect (at 0.2 -2.8702) (size 0.2032 0.8636) (layers "F.Cu" "F.Mask" "F.Paste") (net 18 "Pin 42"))
  (pad "43" smd rect (at -0.2 -2.8702) (size 0.2032 0.8636) (layers "F.Cu" "F.Mask" "F.Paste") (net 19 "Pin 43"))
  (pad "44" smd rect (at -0.599999 -2.8702) (size 0.2032 0.8636) (layers "F.Cu" "F.Mask" "F.Paste") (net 20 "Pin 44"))
  (pad "45" smd rect (at -1.000001 -2.8702) (size 0.2032 0.8636) (layers "F.Cu" "F.Mask" "F.Paste") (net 21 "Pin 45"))
  (pad "46" smd rect (at -1.4 -2.8702) (size 0.2032 0.8636) (layers "F.Cu" "F.Mask" "F.Paste") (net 22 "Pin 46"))
  (pad "47" smd rect (at -1.799999 -2.8702) (size 0.2032 0.8636) (layers "F.Cu" "F.Mask" "F.Paste") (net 23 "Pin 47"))
  (pad "48" smd rect (at -2.200001 -2.8702) (size 0.2032 0.8636) (layers "F.Cu" "F.Mask" "F.Paste") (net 24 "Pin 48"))
  (pad "49" smd rect (at 0 0) (size 4.4958 4.4958) (layers "F.Cu" "F.Mask" "F.Paste") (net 48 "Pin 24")))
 (gr_rect (start 113.03 48.26) (end 185.42 109.22) (stroke (width 0.05) (type default)) (fill no) (layer "Edge.Cuts"))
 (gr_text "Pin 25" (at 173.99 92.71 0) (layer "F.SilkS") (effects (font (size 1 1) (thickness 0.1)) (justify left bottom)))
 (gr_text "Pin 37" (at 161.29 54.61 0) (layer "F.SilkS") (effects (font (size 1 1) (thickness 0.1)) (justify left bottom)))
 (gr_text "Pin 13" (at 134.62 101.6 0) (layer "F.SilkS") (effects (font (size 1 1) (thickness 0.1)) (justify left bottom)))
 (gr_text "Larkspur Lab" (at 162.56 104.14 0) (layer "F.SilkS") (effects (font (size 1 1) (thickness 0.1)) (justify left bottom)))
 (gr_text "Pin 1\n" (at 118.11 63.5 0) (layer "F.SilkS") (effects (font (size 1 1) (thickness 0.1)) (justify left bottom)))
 (segment (start 138.024999 79.145001) (end 125.73 91.44) (width 0.1) (layer "F.Cu") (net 12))
 (segment (start 145.9648 79.155001) (end 145.972202 79.147599) (width 0.2) (layer "F.Cu") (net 12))
 (segment (start 145.9748 79.145001) (end 138.024999 79.145001) (width 0.1) (layer "F.Cu") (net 12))
 (segment (start 145.972202 79.147599) (end 145.9748 79.147599) (width 0.2) (layer "F.Cu") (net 12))
 (segment (start 145.9748 75.145001) (end 134.835001 75.145001) (width 0.1) (layer "F.Cu") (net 2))
 (segment (start 134.835001 75.145001) (end 125.73 66.04) (width 0.1) (layer "F.Cu") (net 2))
 (segment (start 145.9748 75.545) (end 132.695 75.545) (width 0.1) (layer "F.Cu") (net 3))
 (segment (start 132.695 75.545) (end 125.73 68.58) (width 0.1) (layer "F.Cu") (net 3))
 (segment (start 145.9748 75.944999) (end 130.554999 75.944999) (width 0.1) (layer "F.Cu") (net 4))
 (segment (start 130.554999 75.944999) (end 125.73 71.12) (width 0.1) (layer "F.Cu") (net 4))
 (segment (start 145.9748 77.945001) (end 131.604999 77.945001) (width 0.1) (layer "F.Cu") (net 9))
 (segment (start 131.604999 77.945001) (end 125.73 83.82) (width 0.1) (layer "F.Cu") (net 9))
 (segment (start 145.9748 76.745) (end 126.275 76.745) (width 0.1) (layer "F.Cu") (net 6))
 (segment (start 126.275 76.745) (end 125.73 76.2) (width 0.1) (layer "F.Cu") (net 6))
 (segment (start 125.73 76.2) (end 126.279001 76.749001) (width 0.2) (layer "F.Cu") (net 6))
 (segment (start 145.9748 78.744999) (end 135.885001 78.744999) (width 0.1) (layer "F.Cu") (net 11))
 (segment (start 135.885001 78.744999) (end 125.73 88.9) (width 0.1) (layer "F.Cu") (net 11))
 (segment (start 145.9748 78.345) (end 133.745 78.345) (width 0.1) (layer "F.Cu") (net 10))
 (segment (start 133.745 78.345) (end 125.73 86.36) (width 0.1) (layer "F.Cu") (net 10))
 (segment (start 145.9748 76.345001) (end 128.415001 76.345001) (width 0.1) (layer "F.Cu") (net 5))
 (segment (start 128.415001 76.345001) (end 125.73 73.66) (width 0.1) (layer "F.Cu") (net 5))
 (segment (start 127.325 77.145) (end 125.73 78.74) (width 0.1) (layer "F.Cu") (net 7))
 (segment (start 145.9748 77.145) (end 127.325 77.145) (width 0.1) (layer "F.Cu") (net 7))
 (segment (start 136.974999 74.744999) (end 125.73 63.5) (width 0.1) (layer "F.Cu") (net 1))
 (segment (start 145.9748 74.744999) (end 136.974999 74.744999) (width 0.1) (layer "F.Cu") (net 1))
 (segment (start 145.9748 77.544999) (end 129.465001 77.544999) (width 0.1) (layer "F.Cu") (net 8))
 (segment (start 129.465001 77.544999) (end 125.73 81.28) (width 0.1) (layer "F.Cu") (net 8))
 (segment (start 148.245001 79.8152) (end 148.245001 95.594999) (width 0.1) (layer "F.Cu") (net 41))
 (segment (start 148.245001 95.594999) (end 146.05 97.79) (width 0.1) (layer "F.Cu") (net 41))
 (segment (start 150.644999 87.144999) (end 161.29 97.79) (width 0.1) (layer "F.Cu") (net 47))
 (segment (start 150.644999 79.8152) (end 150.644999 87.144999) (width 0.1) (layer "F.Cu") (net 47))
 (segment (start 148.645 79.8152) (end 148.645 97.735) (width 0.1) (layer "F.Cu") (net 42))
 (segment (start 148.645 97.735) (end 148.59 97.79) (width 0.1) (layer "F.Cu") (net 42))
 (segment (start 149.045 95.705) (end 151.13 97.79) (width 0.1) (layer "F.Cu") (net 43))
 (segment (start 149.045 79.8152) (end 149.045 95.705) (width 0.1) (layer "F.Cu") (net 43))
 (segment (start 147.045001 89.174999) (end 138.43 97.79) (width 0.1) (layer "F.Cu") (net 38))
 (segment (start 147.045001 79.8152) (end 147.045001 89.174999) (width 0.1) (layer "F.Cu") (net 38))
 (segment (start 150.245 79.8152) (end 150.245 89.285) (width 0.1) (layer "F.Cu") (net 46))
 (segment (start 150.245 89.285) (end 158.75 97.79) (width 0.1) (layer "F.Cu") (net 46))
 (segment (start 147.844999 79.8152) (end 147.844999 93.455001) (width 0.1) (layer "F.Cu") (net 40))
 (segment (start 147.844999 93.455001) (end 143.51 97.79) (width 0.1) (layer "F.Cu") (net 40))
 (segment (start 149.845001 79.8152) (end 149.845001 91.425001) (width 0.1) (layer "F.Cu") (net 45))
 (segment (start 149.845001 91.425001) (end 156.21 97.79) (width 0.1) (layer "F.Cu") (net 45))
 (segment (start 147.445 79.8152) (end 147.445 91.315) (width 0.1) (layer "F.Cu") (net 39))
 (segment (start 147.445 91.315) (end 140.97 97.79) (width 0.1) (layer "F.Cu") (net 39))
 (segment (start 151.045001 79.8152) (end 151.0324 79.802599) (width 0.1) (layer "F.Cu") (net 48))
 (segment (start 151.0324 79.1324) (end 148.845 76.945) (width 0.1) (layer "F.Cu") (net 48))
 (segment (start 151.045001 79.8152) (end 151.045001 85.005001) (width 0.1) (layer "F.Cu") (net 48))
 (segment (start 151.045001 85.005001) (end 163.83 97.79) (width 0.1) (layer "F.Cu") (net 48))
 (segment (start 151.0324 79.802599) (end 151.0324 79.1324) (width 0.1) (layer "F.Cu") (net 48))
 (segment (start 146.644999 87.035001) (end 135.89 97.79) (width 0.1) (layer "F.Cu") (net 37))
 (segment (start 146.644999 79.8152) (end 146.644999 87.035001) (width 0.1) (layer "F.Cu") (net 37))
 (segment (start 149.444999 93.564999) (end 153.67 97.79) (width 0.1) (layer "F.Cu") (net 44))
 (segment (start 149.444999 79.8152) (end 149.444999 93.564999) (width 0.1) (layer "F.Cu") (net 44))
 (segment (start 151.7152 75.545) (end 164.485 75.545) (width 0.1) (layer "F.Cu") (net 34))
 (segment (start 164.485 75.545) (end 171.45 68.58) (width 0.1) (layer "F.Cu") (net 34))
 (segment (start 168.764999 76.345001) (end 171.45 73.66) (width 0.1) (layer "F.Cu") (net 32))
 (segment (start 151.7152 76.345001) (end 168.764999 76.345001) (width 0.1) (layer "F.Cu") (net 32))
 (segment (start 151.7152 77.945001) (end 165.575001 77.945001) (width 0.1) (layer "F.Cu") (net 28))
 (segment (start 165.575001 77.945001) (end 171.45 83.82) (width 0.1) (layer "F.Cu") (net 28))
 (segment (start 169.855 77.145) (end 171.45 78.74) (width 0.1) (layer "F.Cu") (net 30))
 (segment (start 151.7152 77.145) (end 169.855 77.145) (width 0.1) (layer "F.Cu") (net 30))
 (segment (start 151.7152 78.744999) (end 161.294999 78.744999) (width 0.1) (layer "F.Cu") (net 26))
 (segment (start 161.294999 78.744999) (end 171.45 88.9) (width 0.1) (layer "F.Cu") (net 26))
 (segment (start 151.7152 78.345) (end 163.435 78.345) (width 0.1) (layer "F.Cu") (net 27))
 (segment (start 163.435 78.345) (end 171.45 86.36) (width 0.1) (layer "F.Cu") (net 27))
 (segment (start 162.344999 75.145001) (end 171.45 66.04) (width 0.1) (layer "F.Cu") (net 35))
 (segment (start 151.7152 75.145001) (end 162.344999 75.145001) (width 0.1) (layer "F.Cu") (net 35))
 (segment (start 151.7152 77.544999) (end 167.714999 77.544999) (width 0.1) (layer "F.Cu") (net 29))
 (segment (start 167.714999 77.544999) (end 171.45 81.28) (width 0.1) (layer "F.Cu") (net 29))
 (segment (start 170.905 76.745) (end 171.45 76.2) (width 0.1) (layer "F.Cu") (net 31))
 (segment (start 151.7152 76.745) (end 170.905 76.745) (width 0.1) (layer "F.Cu") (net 31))
 (segment (start 151.7152 75.944999) (end 166.625001 75.944999) (width 0.1) (layer "F.Cu") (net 33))
 (segment (start 166.625001 75.944999) (end 171.45 71.12) (width 0.1) (layer "F.Cu") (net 33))
 (segment (start 160.205001 74.744999) (end 171.45 63.5) (width 0.1) (layer "F.Cu") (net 36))
 (segment (start 151.7152 74.744999) (end 160.205001 74.744999) (width 0.1) (layer "F.Cu") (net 36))
 (segment (start 159.155001 79.145001) (end 171.45 91.44) (width 0.1) (layer "F.Cu") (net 25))
 (segment (start 151.7152 79.145001) (end 159.155001 79.145001) (width 0.1) (layer "F.Cu") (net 25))
 (segment (start 149.444999 60.105001) (end 152.4 57.15) (width 0.1) (layer "F.Cu") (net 17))
 (segment (start 149.444999 74.0748) (end 149.444999 60.105001) (width 0.1) (layer "F.Cu") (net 17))
 (segment (start 146.644999 69.174999) (end 134.62 57.15) (width 0.1) (layer "F.Cu") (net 24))
 (segment (start 146.644999 74.0748) (end 146.644999 69.174999) (width 0.1) (layer "F.Cu") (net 24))
 (segment (start 150.245 74.0748) (end 150.245 64.385) (width 0.1) (layer "F.Cu") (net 15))
 (segment (start 150.245 64.385) (end 157.48 57.15) (width 0.1) (layer "F.Cu") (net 15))
 (segment (start 150.644999 74.0748) (end 150.644999 66.525001) (width 0.1) (layer "F.Cu") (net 14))
 (segment (start 150.644999 66.525001) (end 160.02 57.15) (width 0.1) (layer "F.Cu") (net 14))
 (segment (start 147.844999 62.754999) (end 142.24 57.15) (width 0.1) (layer "F.Cu") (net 21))
 (segment (start 147.844999 74.0748) (end 147.844999 62.754999) (width 0.1) (layer "F.Cu") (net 21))
 (segment (start 149.845001 74.0748) (end 149.845001 62.244999) (width 0.1) (layer "F.Cu") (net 16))
 (segment (start 149.845001 62.244999) (end 154.94 57.15) (width 0.1) (layer "F.Cu") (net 16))
 (segment (start 148.245001 60.615001) (end 144.78 57.15) (width 0.1) (layer "F.Cu") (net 20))
 (segment (start 148.245001 74.0748) (end 148.245001 60.615001) (width 0.1) (layer "F.Cu") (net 20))
 (segment (start 147.445 74.0748) (end 147.445 64.895) (width 0.1) (layer "F.Cu") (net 22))
 (segment (start 147.445 64.895) (end 139.7 57.15) (width 0.1) (layer "F.Cu") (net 22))
 (segment (start 148.645 74.0748) (end 148.645 58.475) (width 0.1) (layer "F.Cu") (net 19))
 (segment (start 148.645 58.475) (end 147.32 57.15) (width 0.1) (layer "F.Cu") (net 19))
 (segment (start 147.045001 74.0748) (end 147.045001 67.035001) (width 0.1) (layer "F.Cu") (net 23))
 (segment (start 147.045001 67.035001) (end 137.16 57.15) (width 0.1) (layer "F.Cu") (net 23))
 (segment (start 149.045 57.965) (end 149.86 57.15) (width 0.1) (layer "F.Cu") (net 18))
 (segment (start 149.045 74.0748) (end 149.045 57.965) (width 0.1) (layer "F.Cu") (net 18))
 (segment (start 151.045001 74.0748) (end 151.045001 68.664999) (width 0.1) (layer "F.Cu") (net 13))
 (segment (start 151.045001 68.664999) (end 162.56 57.15) (width 0.1) (layer "F.Cu") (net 13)))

